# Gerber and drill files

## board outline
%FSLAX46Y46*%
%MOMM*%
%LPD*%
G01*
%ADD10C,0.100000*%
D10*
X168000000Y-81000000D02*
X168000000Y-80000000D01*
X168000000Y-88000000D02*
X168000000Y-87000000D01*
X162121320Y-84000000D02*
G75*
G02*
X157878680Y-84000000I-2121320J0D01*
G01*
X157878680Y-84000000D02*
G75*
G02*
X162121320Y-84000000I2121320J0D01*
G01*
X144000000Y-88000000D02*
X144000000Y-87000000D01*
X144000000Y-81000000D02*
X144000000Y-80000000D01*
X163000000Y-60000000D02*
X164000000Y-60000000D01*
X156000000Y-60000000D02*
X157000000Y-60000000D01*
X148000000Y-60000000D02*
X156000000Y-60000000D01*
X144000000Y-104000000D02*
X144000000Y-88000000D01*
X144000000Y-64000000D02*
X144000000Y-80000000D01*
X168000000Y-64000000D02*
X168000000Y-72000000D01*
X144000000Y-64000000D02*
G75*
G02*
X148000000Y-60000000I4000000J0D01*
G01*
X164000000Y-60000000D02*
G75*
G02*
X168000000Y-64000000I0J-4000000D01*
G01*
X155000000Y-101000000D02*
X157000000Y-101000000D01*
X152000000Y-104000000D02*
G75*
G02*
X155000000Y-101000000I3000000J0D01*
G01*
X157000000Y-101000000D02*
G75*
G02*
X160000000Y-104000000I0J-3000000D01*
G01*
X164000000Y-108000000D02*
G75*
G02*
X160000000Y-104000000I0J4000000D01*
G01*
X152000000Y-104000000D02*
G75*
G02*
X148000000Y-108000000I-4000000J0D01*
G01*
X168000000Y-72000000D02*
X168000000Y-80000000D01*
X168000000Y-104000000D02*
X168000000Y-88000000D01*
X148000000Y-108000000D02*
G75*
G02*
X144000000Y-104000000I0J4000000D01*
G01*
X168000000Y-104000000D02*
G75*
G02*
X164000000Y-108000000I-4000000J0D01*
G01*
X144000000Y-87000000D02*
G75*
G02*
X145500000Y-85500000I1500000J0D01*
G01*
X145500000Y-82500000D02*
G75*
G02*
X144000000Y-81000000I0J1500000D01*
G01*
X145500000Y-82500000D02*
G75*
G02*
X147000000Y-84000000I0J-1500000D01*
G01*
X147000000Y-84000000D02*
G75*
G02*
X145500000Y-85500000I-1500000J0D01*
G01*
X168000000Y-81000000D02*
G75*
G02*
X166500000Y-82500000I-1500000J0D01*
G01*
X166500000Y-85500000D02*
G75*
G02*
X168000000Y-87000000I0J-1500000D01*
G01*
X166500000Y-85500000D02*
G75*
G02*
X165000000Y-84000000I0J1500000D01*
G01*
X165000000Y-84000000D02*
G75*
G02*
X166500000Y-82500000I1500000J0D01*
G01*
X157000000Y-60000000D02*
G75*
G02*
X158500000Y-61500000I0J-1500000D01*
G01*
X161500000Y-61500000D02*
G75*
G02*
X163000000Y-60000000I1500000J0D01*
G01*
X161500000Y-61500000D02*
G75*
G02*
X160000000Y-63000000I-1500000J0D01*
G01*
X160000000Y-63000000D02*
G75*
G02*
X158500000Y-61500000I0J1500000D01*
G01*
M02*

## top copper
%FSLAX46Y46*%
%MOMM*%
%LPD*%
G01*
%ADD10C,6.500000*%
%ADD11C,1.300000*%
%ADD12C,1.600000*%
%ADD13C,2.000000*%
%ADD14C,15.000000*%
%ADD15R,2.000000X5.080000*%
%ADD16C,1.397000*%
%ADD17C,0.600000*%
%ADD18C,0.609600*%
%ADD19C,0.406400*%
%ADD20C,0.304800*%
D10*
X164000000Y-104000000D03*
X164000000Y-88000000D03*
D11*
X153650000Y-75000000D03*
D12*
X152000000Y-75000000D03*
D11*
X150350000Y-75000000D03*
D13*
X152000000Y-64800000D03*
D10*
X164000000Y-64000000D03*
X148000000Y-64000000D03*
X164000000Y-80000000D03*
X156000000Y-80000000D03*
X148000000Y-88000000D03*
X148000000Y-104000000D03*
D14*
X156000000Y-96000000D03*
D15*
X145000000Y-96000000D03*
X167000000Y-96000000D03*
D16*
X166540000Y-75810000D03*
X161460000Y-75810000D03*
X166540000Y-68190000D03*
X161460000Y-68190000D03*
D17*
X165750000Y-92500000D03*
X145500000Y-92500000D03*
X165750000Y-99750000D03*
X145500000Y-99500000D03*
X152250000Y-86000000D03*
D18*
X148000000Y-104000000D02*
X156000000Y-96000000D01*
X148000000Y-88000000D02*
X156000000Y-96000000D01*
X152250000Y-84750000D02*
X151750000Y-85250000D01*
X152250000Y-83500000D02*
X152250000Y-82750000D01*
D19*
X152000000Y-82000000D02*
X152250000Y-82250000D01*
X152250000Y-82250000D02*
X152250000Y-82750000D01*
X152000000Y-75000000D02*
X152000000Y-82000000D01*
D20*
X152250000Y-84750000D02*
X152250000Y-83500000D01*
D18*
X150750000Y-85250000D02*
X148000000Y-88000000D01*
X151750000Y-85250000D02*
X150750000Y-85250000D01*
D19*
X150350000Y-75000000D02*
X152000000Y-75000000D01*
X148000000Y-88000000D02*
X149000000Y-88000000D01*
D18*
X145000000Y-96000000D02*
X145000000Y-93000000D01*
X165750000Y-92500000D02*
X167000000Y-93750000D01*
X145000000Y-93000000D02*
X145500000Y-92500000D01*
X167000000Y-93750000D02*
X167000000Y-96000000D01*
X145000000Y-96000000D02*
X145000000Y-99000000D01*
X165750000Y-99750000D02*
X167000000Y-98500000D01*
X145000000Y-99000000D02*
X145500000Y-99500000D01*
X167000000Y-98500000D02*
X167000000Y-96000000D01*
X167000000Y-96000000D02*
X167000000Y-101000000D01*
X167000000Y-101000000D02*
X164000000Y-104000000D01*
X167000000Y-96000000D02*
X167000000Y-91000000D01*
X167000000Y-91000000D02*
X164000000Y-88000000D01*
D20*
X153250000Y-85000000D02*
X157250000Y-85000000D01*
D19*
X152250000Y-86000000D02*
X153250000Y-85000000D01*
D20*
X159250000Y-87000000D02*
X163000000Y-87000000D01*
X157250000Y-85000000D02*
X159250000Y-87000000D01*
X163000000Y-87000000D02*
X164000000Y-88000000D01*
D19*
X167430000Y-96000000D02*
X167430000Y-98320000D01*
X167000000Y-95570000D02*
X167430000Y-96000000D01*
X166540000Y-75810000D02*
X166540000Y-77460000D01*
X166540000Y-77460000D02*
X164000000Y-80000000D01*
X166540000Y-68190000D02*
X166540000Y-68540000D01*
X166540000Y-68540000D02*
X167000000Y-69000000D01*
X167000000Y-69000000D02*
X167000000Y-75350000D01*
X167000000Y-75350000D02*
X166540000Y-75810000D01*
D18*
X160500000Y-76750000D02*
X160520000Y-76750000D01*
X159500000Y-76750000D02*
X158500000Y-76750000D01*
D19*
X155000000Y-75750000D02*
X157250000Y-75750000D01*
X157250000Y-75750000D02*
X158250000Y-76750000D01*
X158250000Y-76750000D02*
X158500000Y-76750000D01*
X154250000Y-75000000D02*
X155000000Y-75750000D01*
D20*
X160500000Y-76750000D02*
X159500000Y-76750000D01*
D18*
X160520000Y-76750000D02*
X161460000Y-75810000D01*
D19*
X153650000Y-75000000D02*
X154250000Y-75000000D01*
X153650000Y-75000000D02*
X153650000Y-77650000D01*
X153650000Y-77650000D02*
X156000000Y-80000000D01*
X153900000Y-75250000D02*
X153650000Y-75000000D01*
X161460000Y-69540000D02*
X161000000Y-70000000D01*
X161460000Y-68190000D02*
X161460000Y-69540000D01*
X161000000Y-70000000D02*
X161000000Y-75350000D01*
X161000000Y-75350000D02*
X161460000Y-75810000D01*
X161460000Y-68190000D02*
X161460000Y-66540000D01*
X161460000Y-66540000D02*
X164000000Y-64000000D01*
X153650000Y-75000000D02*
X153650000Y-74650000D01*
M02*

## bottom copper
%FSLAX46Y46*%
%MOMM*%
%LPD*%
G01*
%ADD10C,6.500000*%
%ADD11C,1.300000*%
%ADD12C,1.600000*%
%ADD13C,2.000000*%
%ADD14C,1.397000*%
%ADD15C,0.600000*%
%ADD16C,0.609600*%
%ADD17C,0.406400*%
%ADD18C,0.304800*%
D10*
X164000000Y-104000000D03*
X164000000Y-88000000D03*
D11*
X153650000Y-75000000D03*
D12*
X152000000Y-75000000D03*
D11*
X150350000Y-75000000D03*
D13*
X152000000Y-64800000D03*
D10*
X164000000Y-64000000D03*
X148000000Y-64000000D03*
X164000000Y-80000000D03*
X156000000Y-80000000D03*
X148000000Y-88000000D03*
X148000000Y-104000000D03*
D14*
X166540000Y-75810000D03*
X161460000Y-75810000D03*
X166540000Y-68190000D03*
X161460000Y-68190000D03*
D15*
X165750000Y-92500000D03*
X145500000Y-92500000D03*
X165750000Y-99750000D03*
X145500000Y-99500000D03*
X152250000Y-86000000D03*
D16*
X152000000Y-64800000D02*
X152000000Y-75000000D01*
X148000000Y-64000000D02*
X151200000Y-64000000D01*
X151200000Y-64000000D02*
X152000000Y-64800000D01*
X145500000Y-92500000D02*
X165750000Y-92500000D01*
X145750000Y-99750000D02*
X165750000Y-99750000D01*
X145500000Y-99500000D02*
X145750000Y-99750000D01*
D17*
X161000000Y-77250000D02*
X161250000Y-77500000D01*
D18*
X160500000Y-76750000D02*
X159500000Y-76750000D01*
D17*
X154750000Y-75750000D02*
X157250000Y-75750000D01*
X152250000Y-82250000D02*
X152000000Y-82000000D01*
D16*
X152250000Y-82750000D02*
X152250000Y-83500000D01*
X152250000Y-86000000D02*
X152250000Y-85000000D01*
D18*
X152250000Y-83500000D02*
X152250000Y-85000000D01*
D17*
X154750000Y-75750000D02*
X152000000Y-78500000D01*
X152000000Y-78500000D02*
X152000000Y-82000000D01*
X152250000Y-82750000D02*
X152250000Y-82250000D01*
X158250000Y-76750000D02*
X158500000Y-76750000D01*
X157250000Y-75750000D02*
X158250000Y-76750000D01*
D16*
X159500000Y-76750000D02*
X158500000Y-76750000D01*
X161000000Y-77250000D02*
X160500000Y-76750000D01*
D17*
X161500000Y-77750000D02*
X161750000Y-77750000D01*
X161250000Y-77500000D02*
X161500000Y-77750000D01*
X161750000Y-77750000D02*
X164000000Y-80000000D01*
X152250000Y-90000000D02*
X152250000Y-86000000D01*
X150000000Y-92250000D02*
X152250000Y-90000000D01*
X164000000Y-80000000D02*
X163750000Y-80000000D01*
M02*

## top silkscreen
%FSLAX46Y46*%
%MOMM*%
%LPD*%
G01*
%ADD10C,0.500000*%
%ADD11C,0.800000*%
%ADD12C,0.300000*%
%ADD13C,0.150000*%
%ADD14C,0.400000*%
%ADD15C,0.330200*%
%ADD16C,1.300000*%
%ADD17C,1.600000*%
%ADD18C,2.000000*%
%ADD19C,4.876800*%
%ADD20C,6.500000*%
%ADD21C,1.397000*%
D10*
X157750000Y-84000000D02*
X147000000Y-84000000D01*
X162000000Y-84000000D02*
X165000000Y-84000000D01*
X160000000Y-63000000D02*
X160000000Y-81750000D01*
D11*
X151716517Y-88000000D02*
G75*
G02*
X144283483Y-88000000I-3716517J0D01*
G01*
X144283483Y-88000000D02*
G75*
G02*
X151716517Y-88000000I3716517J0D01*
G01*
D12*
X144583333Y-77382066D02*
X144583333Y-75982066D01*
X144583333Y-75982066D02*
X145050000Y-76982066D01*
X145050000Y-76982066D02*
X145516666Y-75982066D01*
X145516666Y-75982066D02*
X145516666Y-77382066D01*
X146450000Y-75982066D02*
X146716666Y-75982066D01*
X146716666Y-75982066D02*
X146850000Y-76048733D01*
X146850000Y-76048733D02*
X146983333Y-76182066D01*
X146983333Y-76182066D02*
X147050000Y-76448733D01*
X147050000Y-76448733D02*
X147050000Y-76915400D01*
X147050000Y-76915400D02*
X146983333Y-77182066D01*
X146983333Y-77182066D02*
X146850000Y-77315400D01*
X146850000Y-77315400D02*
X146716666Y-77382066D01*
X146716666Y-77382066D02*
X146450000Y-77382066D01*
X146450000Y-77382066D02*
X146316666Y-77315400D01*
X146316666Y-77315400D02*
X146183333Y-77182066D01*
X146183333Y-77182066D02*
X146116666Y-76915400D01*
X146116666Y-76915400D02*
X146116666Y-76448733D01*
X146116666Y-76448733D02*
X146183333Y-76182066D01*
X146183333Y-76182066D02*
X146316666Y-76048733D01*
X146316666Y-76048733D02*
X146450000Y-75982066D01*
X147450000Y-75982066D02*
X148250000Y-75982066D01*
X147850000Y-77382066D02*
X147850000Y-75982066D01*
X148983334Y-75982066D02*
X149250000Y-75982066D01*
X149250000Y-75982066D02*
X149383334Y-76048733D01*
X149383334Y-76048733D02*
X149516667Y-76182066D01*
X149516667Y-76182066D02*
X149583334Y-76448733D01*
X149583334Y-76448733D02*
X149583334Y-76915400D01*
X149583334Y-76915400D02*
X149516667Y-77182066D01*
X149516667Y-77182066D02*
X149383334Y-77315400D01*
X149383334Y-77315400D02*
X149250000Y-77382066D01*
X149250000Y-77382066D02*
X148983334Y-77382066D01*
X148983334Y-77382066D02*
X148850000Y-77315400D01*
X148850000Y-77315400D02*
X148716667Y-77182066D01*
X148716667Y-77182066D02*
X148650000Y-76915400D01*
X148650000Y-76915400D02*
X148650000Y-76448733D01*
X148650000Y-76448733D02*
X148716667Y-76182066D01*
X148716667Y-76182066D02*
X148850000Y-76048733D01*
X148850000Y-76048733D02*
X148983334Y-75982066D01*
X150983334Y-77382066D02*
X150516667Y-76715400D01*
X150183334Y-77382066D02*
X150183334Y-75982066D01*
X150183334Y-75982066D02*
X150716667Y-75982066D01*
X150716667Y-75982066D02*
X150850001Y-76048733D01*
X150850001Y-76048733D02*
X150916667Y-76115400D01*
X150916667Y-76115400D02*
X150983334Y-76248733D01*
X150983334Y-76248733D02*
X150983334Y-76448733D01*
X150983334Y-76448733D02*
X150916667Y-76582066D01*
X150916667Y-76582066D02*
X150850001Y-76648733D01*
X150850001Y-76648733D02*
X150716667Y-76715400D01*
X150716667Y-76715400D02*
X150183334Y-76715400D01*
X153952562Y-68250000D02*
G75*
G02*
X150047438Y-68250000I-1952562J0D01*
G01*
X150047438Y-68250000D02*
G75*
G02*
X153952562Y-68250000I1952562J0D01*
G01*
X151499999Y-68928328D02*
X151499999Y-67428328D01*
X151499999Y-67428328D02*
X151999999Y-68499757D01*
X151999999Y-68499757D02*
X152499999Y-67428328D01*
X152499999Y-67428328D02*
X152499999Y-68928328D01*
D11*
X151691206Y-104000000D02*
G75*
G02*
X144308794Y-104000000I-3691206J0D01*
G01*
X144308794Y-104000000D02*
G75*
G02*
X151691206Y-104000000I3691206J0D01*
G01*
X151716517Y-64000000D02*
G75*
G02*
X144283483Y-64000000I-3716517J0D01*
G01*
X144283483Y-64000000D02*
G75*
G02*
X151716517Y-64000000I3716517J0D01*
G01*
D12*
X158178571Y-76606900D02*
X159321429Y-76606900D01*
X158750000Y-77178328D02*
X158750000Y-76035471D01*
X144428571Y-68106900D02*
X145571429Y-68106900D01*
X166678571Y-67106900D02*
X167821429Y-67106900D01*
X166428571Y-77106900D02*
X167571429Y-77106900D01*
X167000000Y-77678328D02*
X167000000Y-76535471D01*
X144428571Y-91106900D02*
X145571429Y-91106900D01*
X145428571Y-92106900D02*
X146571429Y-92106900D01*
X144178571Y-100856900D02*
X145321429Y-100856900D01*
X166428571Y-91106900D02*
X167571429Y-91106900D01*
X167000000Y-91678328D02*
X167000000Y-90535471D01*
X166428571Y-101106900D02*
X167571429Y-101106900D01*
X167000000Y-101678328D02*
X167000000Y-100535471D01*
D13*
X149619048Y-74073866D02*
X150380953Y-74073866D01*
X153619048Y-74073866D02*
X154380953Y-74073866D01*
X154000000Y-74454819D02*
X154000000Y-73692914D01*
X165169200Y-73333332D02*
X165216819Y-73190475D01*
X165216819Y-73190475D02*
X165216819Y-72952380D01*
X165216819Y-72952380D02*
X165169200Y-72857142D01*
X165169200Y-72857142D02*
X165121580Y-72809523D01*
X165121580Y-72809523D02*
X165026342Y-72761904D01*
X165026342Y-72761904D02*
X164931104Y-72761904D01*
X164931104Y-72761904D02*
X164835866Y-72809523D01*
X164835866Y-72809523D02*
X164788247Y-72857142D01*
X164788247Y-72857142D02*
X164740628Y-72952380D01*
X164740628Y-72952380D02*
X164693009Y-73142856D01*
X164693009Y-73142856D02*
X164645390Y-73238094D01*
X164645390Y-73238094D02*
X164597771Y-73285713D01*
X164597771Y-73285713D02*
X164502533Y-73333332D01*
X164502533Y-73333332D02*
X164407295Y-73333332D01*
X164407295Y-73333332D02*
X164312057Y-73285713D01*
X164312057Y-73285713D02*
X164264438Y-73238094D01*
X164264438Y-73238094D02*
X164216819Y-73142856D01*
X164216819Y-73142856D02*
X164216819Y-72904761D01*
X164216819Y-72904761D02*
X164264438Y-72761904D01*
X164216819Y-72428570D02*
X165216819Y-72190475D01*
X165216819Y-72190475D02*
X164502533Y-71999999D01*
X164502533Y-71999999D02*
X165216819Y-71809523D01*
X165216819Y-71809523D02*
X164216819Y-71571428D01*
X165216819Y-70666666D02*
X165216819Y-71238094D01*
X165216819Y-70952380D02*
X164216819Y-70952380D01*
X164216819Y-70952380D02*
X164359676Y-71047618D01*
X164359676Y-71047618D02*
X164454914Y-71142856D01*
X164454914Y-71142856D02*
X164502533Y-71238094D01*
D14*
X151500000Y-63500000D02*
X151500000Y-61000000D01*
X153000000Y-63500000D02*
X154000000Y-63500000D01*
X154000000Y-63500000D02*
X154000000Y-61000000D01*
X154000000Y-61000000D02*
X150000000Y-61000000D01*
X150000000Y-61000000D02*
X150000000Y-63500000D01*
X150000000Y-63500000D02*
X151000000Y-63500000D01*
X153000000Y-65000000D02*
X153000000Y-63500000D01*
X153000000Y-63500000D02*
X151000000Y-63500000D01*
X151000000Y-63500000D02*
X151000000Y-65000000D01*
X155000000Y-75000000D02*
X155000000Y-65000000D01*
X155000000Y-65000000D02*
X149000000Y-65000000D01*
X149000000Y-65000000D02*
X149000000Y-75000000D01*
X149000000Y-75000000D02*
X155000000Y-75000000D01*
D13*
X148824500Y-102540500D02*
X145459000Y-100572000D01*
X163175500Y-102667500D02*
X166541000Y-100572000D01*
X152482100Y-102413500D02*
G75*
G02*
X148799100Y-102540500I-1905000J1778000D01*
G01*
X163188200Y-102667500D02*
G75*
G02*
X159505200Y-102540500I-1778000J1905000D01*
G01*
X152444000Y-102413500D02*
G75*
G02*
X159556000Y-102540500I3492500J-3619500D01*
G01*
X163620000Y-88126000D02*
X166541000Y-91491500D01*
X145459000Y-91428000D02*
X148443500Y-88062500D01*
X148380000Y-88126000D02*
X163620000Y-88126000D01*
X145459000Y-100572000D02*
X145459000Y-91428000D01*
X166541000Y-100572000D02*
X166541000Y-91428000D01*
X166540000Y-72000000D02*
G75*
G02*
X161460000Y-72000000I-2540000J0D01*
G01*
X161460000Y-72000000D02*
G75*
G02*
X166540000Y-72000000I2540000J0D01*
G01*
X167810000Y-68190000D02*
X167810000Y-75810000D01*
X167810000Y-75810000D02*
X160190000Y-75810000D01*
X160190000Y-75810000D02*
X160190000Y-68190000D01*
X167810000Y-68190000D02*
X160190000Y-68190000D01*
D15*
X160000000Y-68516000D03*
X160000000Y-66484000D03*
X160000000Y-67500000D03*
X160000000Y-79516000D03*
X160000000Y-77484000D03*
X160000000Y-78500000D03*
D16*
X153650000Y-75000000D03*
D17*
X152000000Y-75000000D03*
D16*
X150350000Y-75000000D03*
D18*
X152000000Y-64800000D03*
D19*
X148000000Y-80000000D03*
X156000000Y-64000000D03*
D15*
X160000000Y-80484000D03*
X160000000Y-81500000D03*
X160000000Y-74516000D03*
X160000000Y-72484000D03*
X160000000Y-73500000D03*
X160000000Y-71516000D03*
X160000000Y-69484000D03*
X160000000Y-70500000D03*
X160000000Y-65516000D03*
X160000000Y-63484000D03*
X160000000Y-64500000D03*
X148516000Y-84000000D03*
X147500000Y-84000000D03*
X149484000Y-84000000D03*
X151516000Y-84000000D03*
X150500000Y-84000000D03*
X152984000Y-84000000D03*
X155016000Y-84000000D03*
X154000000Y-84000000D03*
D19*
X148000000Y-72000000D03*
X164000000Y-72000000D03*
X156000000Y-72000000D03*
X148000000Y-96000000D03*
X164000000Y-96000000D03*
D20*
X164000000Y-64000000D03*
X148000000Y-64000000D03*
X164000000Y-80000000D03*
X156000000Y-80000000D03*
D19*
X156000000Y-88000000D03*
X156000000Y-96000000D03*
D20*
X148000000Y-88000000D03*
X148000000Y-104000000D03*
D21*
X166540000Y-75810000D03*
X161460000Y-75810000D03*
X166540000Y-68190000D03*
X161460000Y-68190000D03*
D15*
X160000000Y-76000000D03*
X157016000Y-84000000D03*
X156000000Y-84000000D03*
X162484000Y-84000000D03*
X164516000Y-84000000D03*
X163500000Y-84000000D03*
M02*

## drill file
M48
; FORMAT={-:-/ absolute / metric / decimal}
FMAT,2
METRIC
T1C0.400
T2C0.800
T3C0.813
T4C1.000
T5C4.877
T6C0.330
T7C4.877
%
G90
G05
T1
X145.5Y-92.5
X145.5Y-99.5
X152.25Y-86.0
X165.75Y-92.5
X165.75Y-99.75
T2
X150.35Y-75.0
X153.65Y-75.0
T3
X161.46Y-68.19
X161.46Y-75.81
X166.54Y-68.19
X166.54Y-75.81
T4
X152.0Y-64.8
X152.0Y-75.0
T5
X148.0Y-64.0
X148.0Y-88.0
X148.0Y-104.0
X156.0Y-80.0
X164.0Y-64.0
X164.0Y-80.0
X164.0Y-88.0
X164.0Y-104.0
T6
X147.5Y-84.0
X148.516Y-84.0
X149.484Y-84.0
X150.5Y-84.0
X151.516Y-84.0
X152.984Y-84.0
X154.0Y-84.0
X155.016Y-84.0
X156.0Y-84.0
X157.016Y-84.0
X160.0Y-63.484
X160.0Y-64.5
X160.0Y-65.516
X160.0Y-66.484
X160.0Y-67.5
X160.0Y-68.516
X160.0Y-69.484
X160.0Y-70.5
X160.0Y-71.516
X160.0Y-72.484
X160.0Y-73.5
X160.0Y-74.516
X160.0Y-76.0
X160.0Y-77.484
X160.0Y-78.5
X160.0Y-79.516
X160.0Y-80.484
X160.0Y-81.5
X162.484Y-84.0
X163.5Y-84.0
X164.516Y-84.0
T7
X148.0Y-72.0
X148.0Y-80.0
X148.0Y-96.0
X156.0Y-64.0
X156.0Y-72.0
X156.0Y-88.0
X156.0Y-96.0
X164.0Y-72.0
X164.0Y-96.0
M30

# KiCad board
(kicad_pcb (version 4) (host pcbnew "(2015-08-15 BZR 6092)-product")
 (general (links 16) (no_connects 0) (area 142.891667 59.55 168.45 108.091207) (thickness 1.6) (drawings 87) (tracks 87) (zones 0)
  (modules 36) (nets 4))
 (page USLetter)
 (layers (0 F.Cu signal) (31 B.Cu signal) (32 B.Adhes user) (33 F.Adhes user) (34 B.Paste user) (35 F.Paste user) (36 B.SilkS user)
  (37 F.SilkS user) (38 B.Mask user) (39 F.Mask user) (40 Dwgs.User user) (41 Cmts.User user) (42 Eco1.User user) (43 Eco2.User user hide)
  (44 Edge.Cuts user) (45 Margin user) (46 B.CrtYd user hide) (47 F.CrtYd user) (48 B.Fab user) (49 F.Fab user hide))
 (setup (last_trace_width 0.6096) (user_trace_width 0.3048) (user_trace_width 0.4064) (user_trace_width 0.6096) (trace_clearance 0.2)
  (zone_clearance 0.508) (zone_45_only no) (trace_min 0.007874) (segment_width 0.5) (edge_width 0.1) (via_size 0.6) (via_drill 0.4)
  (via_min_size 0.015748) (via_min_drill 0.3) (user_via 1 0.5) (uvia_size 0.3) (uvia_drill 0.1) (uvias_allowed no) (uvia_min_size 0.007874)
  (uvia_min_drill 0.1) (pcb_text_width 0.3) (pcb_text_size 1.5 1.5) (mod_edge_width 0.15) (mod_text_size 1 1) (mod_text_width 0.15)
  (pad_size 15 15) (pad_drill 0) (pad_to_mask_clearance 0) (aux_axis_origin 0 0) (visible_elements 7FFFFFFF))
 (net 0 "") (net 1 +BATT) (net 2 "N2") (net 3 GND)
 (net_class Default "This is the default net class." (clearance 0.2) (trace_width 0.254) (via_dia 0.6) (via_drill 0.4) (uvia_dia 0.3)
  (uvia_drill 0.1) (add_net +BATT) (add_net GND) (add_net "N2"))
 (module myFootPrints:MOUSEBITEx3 (layer F.Cu) (at 160 67.5 90)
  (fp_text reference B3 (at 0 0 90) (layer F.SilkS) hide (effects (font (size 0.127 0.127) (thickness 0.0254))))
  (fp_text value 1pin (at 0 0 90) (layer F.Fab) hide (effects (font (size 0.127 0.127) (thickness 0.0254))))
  (pad "" np_thru_hole circle (at -1.016 0 90) (size 0.3302 0.3302) (drill 0.3302) (layers *.Cu *.Mask F.SilkS))
  (pad "" np_thru_hole circle (at 1.016 0 90) (size 0.3302 0.3302) (drill 0.3302) (layers *.Cu *.Mask F.SilkS))
  (pad "" np_thru_hole circle (at 0 0 90) (size 0.3302 0.3302) (drill 0.3302) (layers *.Cu *.Mask F.SilkS)))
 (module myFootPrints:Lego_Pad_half (layer F.Cu) (at 164 104 180)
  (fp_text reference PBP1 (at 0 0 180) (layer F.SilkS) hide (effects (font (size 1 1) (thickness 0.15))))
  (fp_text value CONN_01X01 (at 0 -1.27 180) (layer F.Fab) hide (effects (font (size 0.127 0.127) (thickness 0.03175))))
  (pad 1 thru_hole circle (at 0 0 180) (size 6.5 6.5) (drill 4.8768) (layers *.Cu B.SilkS B.Mask) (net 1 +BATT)))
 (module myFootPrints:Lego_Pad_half (layer F.Cu) (at 164 88 270)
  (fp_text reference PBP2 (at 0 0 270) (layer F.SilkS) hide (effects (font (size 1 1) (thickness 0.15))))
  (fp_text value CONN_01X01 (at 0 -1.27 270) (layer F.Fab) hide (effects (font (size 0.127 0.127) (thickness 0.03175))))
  (pad 1 thru_hole circle (at 0 0 270) (size 6.5 6.5) (drill 4.8768) (layers *.Cu B.SilkS B.Mask) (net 1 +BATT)))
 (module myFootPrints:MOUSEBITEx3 (layer F.Cu) (at 160 78.5 90)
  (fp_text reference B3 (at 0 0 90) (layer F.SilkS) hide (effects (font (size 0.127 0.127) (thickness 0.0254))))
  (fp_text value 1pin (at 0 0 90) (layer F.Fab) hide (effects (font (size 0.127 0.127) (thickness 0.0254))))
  (pad "" np_thru_hole circle (at -1.016 0 90) (size 0.3302 0.3302) (drill 0.3302) (layers *.Cu *.Mask F.SilkS))
  (pad "" np_thru_hole circle (at 1.016 0 90) (size 0.3302 0.3302) (drill 0.3302) (layers *.Cu *.Mask F.SilkS))
  (pad "" np_thru_hole circle (at 0 0 90) (size 0.3302 0.3302) (drill 0.3302) (layers *.Cu *.Mask F.SilkS)))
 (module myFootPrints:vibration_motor (layer F.Cu) (at 152 70 180)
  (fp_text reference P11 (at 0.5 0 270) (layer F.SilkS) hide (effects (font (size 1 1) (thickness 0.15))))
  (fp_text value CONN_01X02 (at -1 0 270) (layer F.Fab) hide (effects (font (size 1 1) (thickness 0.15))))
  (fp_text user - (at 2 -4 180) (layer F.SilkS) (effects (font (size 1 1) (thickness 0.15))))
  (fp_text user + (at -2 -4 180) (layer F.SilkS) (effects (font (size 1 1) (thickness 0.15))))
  (fp_line (start 0.5 6.5) (end 0.5 9) (layer F.SilkS) (width 0.4))
  (fp_line (start -1 6.5) (end -2 6.5) (layer F.SilkS) (width 0.4))
  (fp_line (start -2 6.5) (end -2 9) (layer F.SilkS) (width 0.4)) (fp_line (start -2 9) (end 2 9) (layer F.SilkS) (width 0.4))
  (fp_line (start 2 9) (end 2 6.5) (layer F.SilkS) (width 0.4))
  (fp_line (start 2 6.5) (end 1 6.5) (layer F.SilkS) (width 0.4))
  (fp_line (start -1 5) (end -1 6.5) (layer F.SilkS) (width 0.4))
  (fp_line (start -1 6.5) (end 1 6.5) (layer F.SilkS) (width 0.4))
  (fp_line (start 1 6.5) (end 1 5) (layer F.SilkS) (width 0.4))
  (fp_line (start -3 -5) (end -3 5) (layer F.SilkS) (width 0.4)) (fp_line (start -3 5) (end 3 5) (layer F.SilkS) (width 0.4))
  (fp_line (start 3 5) (end 3 -5) (layer F.SilkS) (width 0.4))
  (fp_line (start 3 -5) (end -3 -5) (layer F.SilkS) (width 0.4))
  (pad 1 thru_hole circle (at -1.65 -5 180) (size 1.3 1.3) (drill 0.8) (layers *.Cu *.Mask F.SilkS) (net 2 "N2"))
  (pad 2 thru_hole circle (at 0 -5 180) (size 1.6 1.6) (drill 1) (layers *.Cu *.Mask F.SilkS) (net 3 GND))
  (pad 2 thru_hole circle (at 1.65 -5 180) (size 1.3 1.3) (drill 0.8) (layers *.Cu *.Mask F.SilkS) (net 3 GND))
  (pad 2 thru_hole circle (at 0 5.2 180) (size 2 2) (drill 1) (layers *.Cu *.Mask F.SilkS) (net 3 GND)))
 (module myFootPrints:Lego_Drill (layer F.Cu) (at 148 80)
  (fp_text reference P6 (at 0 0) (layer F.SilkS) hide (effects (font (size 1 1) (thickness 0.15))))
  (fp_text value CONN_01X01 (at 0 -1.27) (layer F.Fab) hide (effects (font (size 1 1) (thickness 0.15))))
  (pad "" np_thru_hole circle (at 0 0) (size 4.8768 4.8768) (drill 4.8768) (layers *.Cu *.Mask F.SilkS)))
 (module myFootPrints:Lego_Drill (layer F.Cu) (at 156 64)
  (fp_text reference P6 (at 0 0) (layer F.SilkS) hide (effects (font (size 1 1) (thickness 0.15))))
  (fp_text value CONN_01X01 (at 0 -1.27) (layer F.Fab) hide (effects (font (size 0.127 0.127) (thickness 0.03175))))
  (pad "" np_thru_hole circle (at 0 0) (size 4.8768 4.8768) (drill 4.8768) (layers *.Cu *.Mask F.SilkS)))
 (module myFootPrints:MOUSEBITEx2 (layer F.Cu) (at 160 81.5 90)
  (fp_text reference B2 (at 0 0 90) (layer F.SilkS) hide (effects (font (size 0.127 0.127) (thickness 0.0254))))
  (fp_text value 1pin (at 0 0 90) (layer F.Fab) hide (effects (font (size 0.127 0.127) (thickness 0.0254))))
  (pad "" np_thru_hole circle (at 1.016 0 90) (size 0.3302 0.3302) (drill 0.3302) (layers *.Cu *.Mask F.SilkS))
  (pad "" np_thru_hole circle (at 0 0 90) (size 0.3302 0.3302) (drill 0.3302) (layers *.Cu *.Mask F.SilkS)))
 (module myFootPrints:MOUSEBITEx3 (layer F.Cu) (at 160 73.5 90)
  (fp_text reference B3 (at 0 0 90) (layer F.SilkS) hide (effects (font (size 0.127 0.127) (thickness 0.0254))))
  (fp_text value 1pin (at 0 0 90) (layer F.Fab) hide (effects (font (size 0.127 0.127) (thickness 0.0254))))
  (pad "" np_thru_hole circle (at -1.016 0 90) (size 0.3302 0.3302) (drill 0.3302) (layers *.Cu *.Mask F.SilkS))
  (pad "" np_thru_hole circle (at 1.016 0 90) (size 0.3302 0.3302) (drill 0.3302) (layers *.Cu *.Mask F.SilkS))
  (pad "" np_thru_hole circle (at 0 0 90) (size 0.3302 0.3302) (drill 0.3302) (layers *.Cu *.Mask F.SilkS)))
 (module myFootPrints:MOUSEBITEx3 (layer F.Cu) (at 160 70.5 90)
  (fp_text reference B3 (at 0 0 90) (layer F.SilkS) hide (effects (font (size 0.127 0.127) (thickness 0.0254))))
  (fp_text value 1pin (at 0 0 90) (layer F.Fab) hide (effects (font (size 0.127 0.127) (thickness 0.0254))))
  (pad "" np_thru_hole circle (at -1.016 0 90) (size 0.3302 0.3302) (drill 0.3302) (layers *.Cu *.Mask F.SilkS))
  (pad "" np_thru_hole circle (at 1.016 0 90) (size 0.3302 0.3302) (drill 0.3302) (layers *.Cu *.Mask F.SilkS))
  (pad "" np_thru_hole circle (at 0 0 90) (size 0.3302 0.3302) (drill 0.3302) (layers *.Cu *.Mask F.SilkS)))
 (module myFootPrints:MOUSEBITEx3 (layer F.Cu) (at 160 64.5 90)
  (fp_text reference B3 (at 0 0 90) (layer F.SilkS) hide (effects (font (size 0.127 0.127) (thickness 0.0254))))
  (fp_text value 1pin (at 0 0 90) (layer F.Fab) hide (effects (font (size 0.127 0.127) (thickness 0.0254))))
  (pad "" np_thru_hole circle (at -1.016 0 90) (size 0.3302 0.3302) (drill 0.3302) (layers *.Cu *.Mask F.SilkS))
  (pad "" np_thru_hole circle (at 1.016 0 90) (size 0.3302 0.3302) (drill 0.3302) (layers *.Cu *.Mask F.SilkS))
  (pad "" np_thru_hole circle (at 0 0 90) (size 0.3302 0.3302) (drill 0.3302) (layers *.Cu *.Mask F.SilkS)))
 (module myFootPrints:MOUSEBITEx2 (layer F.Cu) (at 147.5 84)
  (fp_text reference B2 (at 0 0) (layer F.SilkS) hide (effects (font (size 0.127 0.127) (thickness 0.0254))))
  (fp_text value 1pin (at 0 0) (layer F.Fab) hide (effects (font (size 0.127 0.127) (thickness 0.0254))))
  (pad "" np_thru_hole circle (at 1.016 0) (size 0.3302 0.3302) (drill 0.3302) (layers *.Cu *.Mask F.SilkS))
  (pad "" np_thru_hole circle (at 0 0) (size 0.3302 0.3302) (drill 0.3302) (layers *.Cu *.Mask F.SilkS)))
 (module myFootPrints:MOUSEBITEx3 (layer F.Cu) (at 150.5 84)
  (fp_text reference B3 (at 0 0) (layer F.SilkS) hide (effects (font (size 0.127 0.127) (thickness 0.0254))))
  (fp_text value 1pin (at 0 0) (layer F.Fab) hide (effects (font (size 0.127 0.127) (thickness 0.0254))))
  (pad "" np_thru_hole circle (at -1.016 0) (size 0.3302 0.3302) (drill 0.3302) (layers *.Cu *.Mask F.SilkS))
  (pad "" np_thru_hole circle (at 1.016 0) (size 0.3302 0.3302) (drill 0.3302) (layers *.Cu *.Mask F.SilkS))
  (pad "" np_thru_hole circle (at 0 0) (size 0.3302 0.3302) (drill 0.3302) (layers *.Cu *.Mask F.SilkS)))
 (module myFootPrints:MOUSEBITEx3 (layer F.Cu) (at 154 84)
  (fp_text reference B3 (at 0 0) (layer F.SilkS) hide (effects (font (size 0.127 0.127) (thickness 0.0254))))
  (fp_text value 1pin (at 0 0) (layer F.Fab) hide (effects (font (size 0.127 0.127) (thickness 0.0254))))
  (pad "" np_thru_hole circle (at -1.016 0) (size 0.3302 0.3302) (drill 0.3302) (layers *.Cu *.Mask F.SilkS))
  (pad "" np_thru_hole circle (at 1.016 0) (size 0.3302 0.3302) (drill 0.3302) (layers *.Cu *.Mask F.SilkS))
  (pad "" np_thru_hole circle (at 0 0) (size 0.3302 0.3302) (drill 0.3302) (layers *.Cu *.Mask F.SilkS)))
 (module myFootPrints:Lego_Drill (layer F.Cu) (at 148 72)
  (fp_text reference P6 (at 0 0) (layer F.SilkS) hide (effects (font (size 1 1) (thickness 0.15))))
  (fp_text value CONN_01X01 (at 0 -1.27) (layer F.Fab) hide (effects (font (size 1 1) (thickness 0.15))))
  (pad "" np_thru_hole circle (at 0 0) (size 4.8768 4.8768) (drill 4.8768) (layers *.Cu *.Mask F.SilkS)))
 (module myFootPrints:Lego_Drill (layer F.Cu) (at 164 72)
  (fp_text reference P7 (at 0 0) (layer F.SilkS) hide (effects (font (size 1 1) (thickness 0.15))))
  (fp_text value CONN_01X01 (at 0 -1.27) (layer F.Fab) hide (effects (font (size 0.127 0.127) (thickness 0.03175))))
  (pad "" np_thru_hole circle (at 0 0) (size 4.8768 4.8768) (drill 4.8768) (layers *.Cu *.Mask F.SilkS)))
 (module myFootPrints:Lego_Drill (layer F.Cu) (at 156 72)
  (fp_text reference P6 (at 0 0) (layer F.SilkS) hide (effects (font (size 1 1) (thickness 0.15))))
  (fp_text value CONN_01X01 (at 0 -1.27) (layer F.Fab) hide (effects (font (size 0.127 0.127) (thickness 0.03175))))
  (pad "" np_thru_hole circle (at 0 0) (size 4.8768 4.8768) (drill 4.8768) (layers *.Cu *.Mask F.SilkS)))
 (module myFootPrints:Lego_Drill (layer F.Cu) (at 148 96)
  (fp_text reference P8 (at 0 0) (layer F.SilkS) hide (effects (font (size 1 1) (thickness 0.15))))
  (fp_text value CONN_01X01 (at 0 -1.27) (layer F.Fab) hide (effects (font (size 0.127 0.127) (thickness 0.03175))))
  (pad "" np_thru_hole circle (at 0 0) (size 4.8768 4.8768) (drill 4.8768) (layers *.Cu *.Mask F.SilkS)))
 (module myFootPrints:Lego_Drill (layer F.Cu) (at 164 96)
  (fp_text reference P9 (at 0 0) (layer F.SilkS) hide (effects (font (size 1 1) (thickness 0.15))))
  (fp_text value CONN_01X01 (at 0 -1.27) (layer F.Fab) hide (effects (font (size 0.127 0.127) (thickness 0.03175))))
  (pad "" np_thru_hole circle (at 0 0) (size 4.8768 4.8768) (drill 4.8768) (layers *.Cu *.Mask F.SilkS)))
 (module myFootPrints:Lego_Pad (layer F.Cu) (at 164 64)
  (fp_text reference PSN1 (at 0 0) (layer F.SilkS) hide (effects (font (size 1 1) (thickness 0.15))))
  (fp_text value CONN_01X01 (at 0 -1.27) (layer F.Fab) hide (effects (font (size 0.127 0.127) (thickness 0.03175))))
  (pad 1 thru_hole circle (at 0 0) (size 6.5 6.5) (drill 4.8768) (layers *.Cu *.Mask F.SilkS) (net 2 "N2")))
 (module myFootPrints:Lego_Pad (layer F.Cu) (at 148 64)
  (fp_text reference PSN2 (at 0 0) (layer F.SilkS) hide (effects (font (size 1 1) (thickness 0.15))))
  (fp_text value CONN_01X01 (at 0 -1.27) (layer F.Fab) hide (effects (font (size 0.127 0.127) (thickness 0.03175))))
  (pad 1 thru_hole circle (at 0 0) (size 6.5 6.5) (drill 4.8768) (layers *.Cu *.Mask F.SilkS) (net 3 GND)))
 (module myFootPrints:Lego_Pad (layer F.Cu) (at 164 80)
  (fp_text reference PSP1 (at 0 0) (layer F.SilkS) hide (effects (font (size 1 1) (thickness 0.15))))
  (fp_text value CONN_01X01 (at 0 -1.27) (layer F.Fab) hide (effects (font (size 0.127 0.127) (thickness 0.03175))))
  (pad 1 thru_hole circle (at 0 0) (size 6.5 6.5) (drill 4.8768) (layers *.Cu *.Mask F.SilkS) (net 1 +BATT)))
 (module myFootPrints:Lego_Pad (layer F.Cu) (at 156 80)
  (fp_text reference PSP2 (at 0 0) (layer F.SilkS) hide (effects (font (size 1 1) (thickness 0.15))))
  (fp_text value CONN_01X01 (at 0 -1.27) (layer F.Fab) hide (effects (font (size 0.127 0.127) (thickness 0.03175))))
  (pad 1 thru_hole circle (at 0 0) (size 6.5 6.5) (drill 4.8768) (layers *.Cu *.Mask F.SilkS) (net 2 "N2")))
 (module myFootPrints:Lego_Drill (layer F.Cu) (at 156 88)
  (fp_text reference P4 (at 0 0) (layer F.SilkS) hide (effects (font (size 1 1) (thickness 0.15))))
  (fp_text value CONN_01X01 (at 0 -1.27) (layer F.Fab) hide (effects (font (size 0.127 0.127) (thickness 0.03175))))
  (pad "" np_thru_hole circle (at 0 0) (size 4.8768 4.8768) (drill 4.8768) (layers *.Cu *.Mask F.SilkS)))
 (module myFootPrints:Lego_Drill (layer F.Cu) (at 156 96)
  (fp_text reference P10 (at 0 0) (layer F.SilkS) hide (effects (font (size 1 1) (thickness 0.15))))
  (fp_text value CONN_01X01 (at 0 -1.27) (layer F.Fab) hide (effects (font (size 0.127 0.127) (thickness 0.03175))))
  (pad "" np_thru_hole circle (at 0 0) (size 4.8768 4.8768) (drill 4.8768) (layers *.Cu *.Mask F.SilkS)))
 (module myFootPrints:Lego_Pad (layer F.Cu) (at 148 88)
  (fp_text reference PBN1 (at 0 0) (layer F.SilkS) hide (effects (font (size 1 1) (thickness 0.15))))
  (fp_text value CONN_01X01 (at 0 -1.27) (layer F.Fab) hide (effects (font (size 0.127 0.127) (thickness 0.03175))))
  (pad 1 thru_hole circle (at 0 0) (size 6.5 6.5) (drill 4.8768) (layers *.Cu *.Mask F.SilkS) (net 3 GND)))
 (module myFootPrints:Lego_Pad (layer F.Cu) (at 148 104)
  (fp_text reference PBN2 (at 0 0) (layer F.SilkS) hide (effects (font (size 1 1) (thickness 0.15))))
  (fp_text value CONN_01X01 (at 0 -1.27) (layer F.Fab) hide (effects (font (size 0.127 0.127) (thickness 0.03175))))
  (pad 1 thru_hole circle (at 0 0) (size 6.5 6.5) (drill 4.8768) (layers *.Cu *.Mask F.SilkS) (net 3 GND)))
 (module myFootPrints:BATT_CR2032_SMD (layer F.Cu) (at 156 96)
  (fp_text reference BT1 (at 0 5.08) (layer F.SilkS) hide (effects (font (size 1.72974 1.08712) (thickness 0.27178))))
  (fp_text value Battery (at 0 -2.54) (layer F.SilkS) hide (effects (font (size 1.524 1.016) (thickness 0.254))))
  (fp_line (start -7.1755 6.5405) (end -10.541 4.572) (layer F.SilkS) (width 0.15))
  (fp_line (start 7.1755 6.6675) (end 10.541 4.572) (layer F.SilkS) (width 0.15))
  (fp_arc (start -5.4229 4.6355) (end -3.5179 6.4135) (angle 90) (layer F.SilkS) (width 0.15))
  (fp_arc (start 5.4102 4.7625) (end 7.1882 6.6675) (angle 90) (layer F.SilkS) (width 0.15))
  (fp_arc (start -0.0635 10.033) (end -3.556 6.4135) (angle 90) (layer F.SilkS) (width 0.15))
  (fp_line (start 7.62 -7.874) (end 10.541 -4.5085) (layer F.SilkS) (width 0.15))
  (fp_line (start -10.541 -4.572) (end -7.5565 -7.9375) (layer F.SilkS) (width 0.15))
  (fp_line (start -7.62 -7.874) (end 7.62 -7.874) (layer F.SilkS) (width 0.15))
  (fp_line (start -10.541 4.572) (end -10.541 -4.572) (layer F.SilkS) (width 0.15))
  (fp_line (start 10.541 4.572) (end 10.541 -4.572) (layer F.SilkS) (width 0.15))
  (pad 2 smd circle (at 0 0) (size 15 15) (layers F.Cu F.Paste F.Mask) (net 3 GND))
  (pad 1 smd rect (at -11 0) (size 2 5.08) (layers F.Cu F.Paste F.Mask) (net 1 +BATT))
  (pad 1 smd rect (at 11 0) (size 2 5.08) (layers F.Cu F.Paste F.Mask) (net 1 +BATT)))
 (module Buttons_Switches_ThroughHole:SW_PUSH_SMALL (layer F.Cu) (at 164 72 270)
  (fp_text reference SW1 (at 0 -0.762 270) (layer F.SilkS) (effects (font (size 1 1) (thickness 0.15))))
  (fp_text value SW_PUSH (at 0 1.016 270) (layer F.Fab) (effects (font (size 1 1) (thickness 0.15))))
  (fp_circle (center 0 0) (end 0 -2.54) (layer F.SilkS) (width 0.15))
  (fp_line (start -3.81 -3.81) (end 3.81 -3.81) (layer F.SilkS) (width 0.15))
  (fp_line (start 3.81 -3.81) (end 3.81 3.81) (layer F.SilkS) (width 0.15))
  (fp_line (start 3.81 3.81) (end -3.81 3.81) (layer F.SilkS) (width 0.15))
  (fp_line (start -3.81 -3.81) (end -3.81 3.81) (layer F.SilkS) (width 0.15))
  (pad 1 thru_hole circle (at 3.81 -2.54 270) (size 1.397 1.397) (drill 0.8128) (layers *.Cu *.Mask F.SilkS) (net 1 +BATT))
  (pad 2 thru_hole circle (at 3.81 2.54 270) (size 1.397 1.397) (drill 0.8128) (layers *.Cu *.Mask F.SilkS) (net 2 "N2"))
  (pad 1 thru_hole circle (at -3.81 -2.54 270) (size 1.397 1.397) (drill 0.8128) (layers *.Cu *.Mask F.SilkS) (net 1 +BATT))
  (pad 2 thru_hole circle (at -3.81 2.54 270) (size 1.397 1.397) (drill 0.8128) (layers *.Cu *.Mask F.SilkS) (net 2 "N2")))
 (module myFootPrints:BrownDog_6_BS (layer F.Cu) (at 160.4 92.8)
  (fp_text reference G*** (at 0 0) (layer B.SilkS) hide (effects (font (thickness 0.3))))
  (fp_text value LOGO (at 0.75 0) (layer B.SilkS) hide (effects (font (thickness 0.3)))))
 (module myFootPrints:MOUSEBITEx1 (layer F.Cu) (at 160 76)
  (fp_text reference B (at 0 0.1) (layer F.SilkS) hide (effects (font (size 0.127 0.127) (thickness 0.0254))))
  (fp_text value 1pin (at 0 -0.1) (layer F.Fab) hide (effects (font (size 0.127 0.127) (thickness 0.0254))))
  (pad "" np_thru_hole circle (at 0 0) (size 0.3302 0.3302) (drill 0.3302) (layers *.Cu *.Mask F.SilkS)))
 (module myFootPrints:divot (layer F.Cu) (at 144 84 90)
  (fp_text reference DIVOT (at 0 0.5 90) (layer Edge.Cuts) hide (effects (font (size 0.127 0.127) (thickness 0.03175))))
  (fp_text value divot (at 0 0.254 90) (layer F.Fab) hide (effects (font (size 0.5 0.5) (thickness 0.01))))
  (fp_arc (start -3 1.5) (end -3 0) (angle 90) (layer Edge.Cuts) (width 0.1))
  (fp_arc (start 3 1.5) (end 1.5 1.5) (angle 90) (layer Edge.Cuts) (width 0.1))
  (fp_arc (start 0 1.5) (end 1.5 1.5) (angle 90) (layer Edge.Cuts) (width 0.1))
  (fp_arc (start 0 1.5) (end 0 3) (angle 90) (layer Edge.Cuts) (width 0.1)))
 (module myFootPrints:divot (layer F.Cu) (at 168 84 270)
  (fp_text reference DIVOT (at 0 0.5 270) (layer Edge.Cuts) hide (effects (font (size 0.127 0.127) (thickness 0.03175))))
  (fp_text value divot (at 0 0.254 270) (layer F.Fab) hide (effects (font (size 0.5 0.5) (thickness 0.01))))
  (fp_arc (start -3 1.5) (end -3 0) (angle 90) (layer Edge.Cuts) (width 0.1))
  (fp_arc (start 3 1.5) (end 1.5 1.5) (angle 90) (layer Edge.Cuts) (width 0.1))
  (fp_arc (start 0 1.5) (end 1.5 1.5) (angle 90) (layer Edge.Cuts) (width 0.1))
  (fp_arc (start 0 1.5) (end 0 3) (angle 90) (layer Edge.Cuts) (width 0.1)))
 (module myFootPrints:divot (layer F.Cu) (at 160 60)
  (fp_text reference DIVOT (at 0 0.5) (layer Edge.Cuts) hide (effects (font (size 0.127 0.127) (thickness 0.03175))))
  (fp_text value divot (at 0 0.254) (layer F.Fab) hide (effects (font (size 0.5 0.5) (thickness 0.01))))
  (fp_arc (start -3 1.5) (end -3 0) (angle 90) (layer Edge.Cuts) (width 0.1))
  (fp_arc (start 3 1.5) (end 1.5 1.5) (angle 90) (layer Edge.Cuts) (width 0.1))
  (fp_arc (start 0 1.5) (end 1.5 1.5) (angle 90) (layer Edge.Cuts) (width 0.1))
  (fp_arc (start 0 1.5) (end 0 3) (angle 90) (layer Edge.Cuts) (width 0.1)))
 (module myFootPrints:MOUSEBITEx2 (layer F.Cu) (at 156 84)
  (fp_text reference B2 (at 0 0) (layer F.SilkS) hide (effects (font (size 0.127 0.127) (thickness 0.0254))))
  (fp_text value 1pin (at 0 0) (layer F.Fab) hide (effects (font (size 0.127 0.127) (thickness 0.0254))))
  (pad "" np_thru_hole circle (at 1.016 0) (size 0.3302 0.3302) (drill 0.3302) (layers *.Cu *.Mask F.SilkS))
  (pad "" np_thru_hole circle (at 0 0) (size 0.3302 0.3302) (drill 0.3302) (layers *.Cu *.Mask F.SilkS)))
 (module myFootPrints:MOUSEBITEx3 (layer F.Cu) (at 163.5 84)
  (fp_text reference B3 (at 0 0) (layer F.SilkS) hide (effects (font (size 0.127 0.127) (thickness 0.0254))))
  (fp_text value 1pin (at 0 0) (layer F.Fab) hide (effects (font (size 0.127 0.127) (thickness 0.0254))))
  (pad "" np_thru_hole circle (at -1.016 0) (size 0.3302 0.3302) (drill 0.3302) (layers *.Cu *.Mask F.SilkS))
  (pad "" np_thru_hole circle (at 1.016 0) (size 0.3302 0.3302) (drill 0.3302) (layers *.Cu *.Mask F.SilkS))
  (pad "" np_thru_hole circle (at 0 0) (size 0.3302 0.3302) (drill 0.3302) (layers *.Cu *.Mask F.SilkS)))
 (gr_line (start 157.75 84) (end 147 84) (angle 90) (layer F.SilkS) (width 0.5))
 (gr_line (start 162 84) (end 165 84) (angle 90) (layer F.SilkS) (width 0.5))
 (gr_line (start 160 63) (end 160 81.75) (angle 90) (layer F.SilkS) (width 0.5))
 (gr_line (start 168 81) (end 168 80) (angle 90) (layer Edge.Cuts) (width 0.1))
 (gr_line (start 168 88) (end 168 87) (angle 90) (layer Edge.Cuts) (width 0.1))
 (gr_circle (center 160 84) (end 158.5 82.5) (layer Edge.Cuts) (width 0.1))
 (gr_line (start 144 88) (end 144 87) (angle 90) (layer Edge.Cuts) (width 0.1))
 (gr_line (start 144 81) (end 144 80) (angle 90) (layer Edge.Cuts) (width 0.1))
 (gr_circle (center 148 88) (end 144.5 86.75) (layer F.SilkS) (width 0.8))
 (gr_line (start 163 60) (end 164 60) (angle 90) (layer Edge.Cuts) (width 0.1))
 (gr_line (start 156 60) (end 157 60) (angle 90) (layer Edge.Cuts) (width 0.1))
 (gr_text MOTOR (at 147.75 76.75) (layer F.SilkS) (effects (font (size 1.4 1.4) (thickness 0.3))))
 (gr_circle (center 152 68.25) (end 150.5 67) (layer F.SilkS) (width 0.3))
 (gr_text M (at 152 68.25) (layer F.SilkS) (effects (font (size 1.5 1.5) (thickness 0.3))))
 (gr_circle (center 148 104) (end 146.25 100.75) (layer F.SilkS) (width 0.8))
 (gr_circle (center 148 64) (end 146.75 60.5) (layer F.SilkS) (width 0.8))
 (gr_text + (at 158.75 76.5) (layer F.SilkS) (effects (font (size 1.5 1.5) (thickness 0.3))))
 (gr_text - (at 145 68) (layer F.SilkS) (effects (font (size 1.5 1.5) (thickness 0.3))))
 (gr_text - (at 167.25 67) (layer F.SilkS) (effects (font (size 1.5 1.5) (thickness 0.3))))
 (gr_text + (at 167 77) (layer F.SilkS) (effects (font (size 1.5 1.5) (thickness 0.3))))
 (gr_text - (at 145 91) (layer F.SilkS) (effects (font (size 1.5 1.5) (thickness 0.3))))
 (gr_line (start 148 60) (end 156 60) (angle 90) (layer Edge.Cuts) (width 0.1))
 (gr_line (start 144 104) (end 144 88) (angle 90) (layer Edge.Cuts) (width 0.1))
 (gr_line (start 144 64) (end 144 80) (angle 90) (layer Edge.Cuts) (width 0.1))
 (gr_line (start 168 64) (end 168 72) (angle 90) (layer Edge.Cuts) (width 0.1))
 (gr_arc (start 148 64) (end 144 64) (angle 90) (layer Edge.Cuts) (width 0.1))
 (gr_arc (start 164 64) (end 164 60) (angle 90) (layer Edge.Cuts) (width 0.1))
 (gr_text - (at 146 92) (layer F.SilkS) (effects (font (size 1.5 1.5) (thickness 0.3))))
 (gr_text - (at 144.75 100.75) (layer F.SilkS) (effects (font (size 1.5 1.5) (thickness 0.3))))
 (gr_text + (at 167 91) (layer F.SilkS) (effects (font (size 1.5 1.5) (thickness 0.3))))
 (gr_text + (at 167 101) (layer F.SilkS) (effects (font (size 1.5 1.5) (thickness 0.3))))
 (gr_line (start 155 101) (end 157 101) (angle 90) (layer Edge.Cuts) (width 0.1))
 (gr_arc (start 155 104) (end 152 104) (angle 90) (layer Edge.Cuts) (width 0.1))
 (gr_arc (start 157 104) (end 157 101) (angle 90) (layer Edge.Cuts) (width 0.1))
 (gr_arc (start 164 104) (end 164 108) (angle 90) (layer Edge.Cuts) (width 0.1))
 (gr_arc (start 148 104) (end 152 104) (angle 90) (layer Edge.Cuts) (width 0.1))
 (gr_line (start 168 72) (end 168 80) (angle 90) (layer Edge.Cuts) (width 0.1))
 (gr_line (start 168 104) (end 168 88) (angle 90) (layer Edge.Cuts) (width 0.1))
 (gr_arc (start 148 104) (end 148 108) (angle 90) (layer Edge.Cuts) (width 0.1))
 (gr_arc (start 164 104) (end 168 104) (angle 90) (layer Edge.Cuts) (width 0.1))
 (segment (start 148 104) (end 156 96) (width 0.6096) (layer F.Cu) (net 3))
 (segment (start 148 88) (end 156 96) (width 0.6096) (layer F.Cu) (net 3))
 (segment (start 152.25 84.75) (end 151.75 85.25) (width 0.6096) (layer F.Cu) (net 3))
 (segment (start 152.25 83.5) (end 152.25 82.75) (width 0.6096) (layer F.Cu) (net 3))
 (segment (start 152 82) (end 152.25 82.25) (width 0.4064) (layer F.Cu) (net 3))
 (segment (start 152.25 82.25) (end 152.25 82.75) (width 0.4064) (layer F.Cu) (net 3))
 (segment (start 152 75) (end 152 82) (width 0.4064) (layer F.Cu) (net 3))
 (segment (start 152.25 84.75) (end 152.25 83.5) (width 0.3048) (layer F.Cu) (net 3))
 (segment (start 150.75 85.25) (end 148 88) (width 0.6096) (layer F.Cu) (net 3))
 (segment (start 151.75 85.25) (end 150.75 85.25) (width 0.6096) (layer F.Cu) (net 3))
 (segment (start 150.35 75) (end 152 75) (width 0.4064) (layer F.Cu) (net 3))
 (segment (start 152 64.8) (end 152 75) (width 0.6096) (layer B.Cu) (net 3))
 (segment (start 148 64) (end 151.2 64) (width 0.6096) (layer B.Cu) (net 3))
 (segment (start 151.2 64) (end 152 64.8) (width 0.6096) (layer B.Cu) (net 3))
 (segment (start 148 88) (end 149 88) (width 0.4064) (layer F.Cu) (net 3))
 (segment (start 145 96) (end 145 93) (width 0.6096) (layer F.Cu) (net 1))
 (segment (start 165.75 92.5) (end 167 93.75) (width 0.6096) (layer F.Cu) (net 1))
 (via (at 165.75 92.5) (size 0.6) (drill 0.4) (layers F.Cu B.Cu) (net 1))
 (segment (start 145.5 92.5) (end 165.75 92.5) (width 0.6096) (layer B.Cu) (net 1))
 (via (at 145.5 92.5) (size 0.6) (drill 0.4) (layers F.Cu B.Cu) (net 1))
 (segment (start 145 93) (end 145.5 92.5) (width 0.6096) (layer F.Cu) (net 1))
 (segment (start 167 93.75) (end 167 96) (width 0.6096) (layer F.Cu) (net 1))
 (segment (start 145 96) (end 145 99) (width 0.6096) (layer F.Cu) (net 1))
 (segment (start 165.75 99.75) (end 167 98.5) (width 0.6096) (layer F.Cu) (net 1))
 (via (at 165.75 99.75) (size 0.6) (drill 0.4) (layers F.Cu B.Cu) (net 1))
 (segment (start 145.75 99.75) (end 165.75 99.75) (width 0.6096) (layer B.Cu) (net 1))
 (segment (start 145.5 99.5) (end 145.75 99.75) (width 0.6096) (layer B.Cu) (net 1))
 (via (at 145.5 99.5) (size 0.6) (drill 0.4) (layers F.Cu B.Cu) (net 1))
 (segment (start 145 99) (end 145.5 99.5) (width 0.6096) (layer F.Cu) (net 1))
 (segment (start 167 98.5) (end 167 96) (width 0.6096) (layer F.Cu) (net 1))
 (segment (start 167 96) (end 167 101) (width 0.6096) (layer F.Cu) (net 1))
 (segment (start 167 101) (end 164 104) (width 0.6096) (layer F.Cu) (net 1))
 (segment (start 167 96) (end 167 91) (width 0.6096) (layer F.Cu) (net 1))
 (segment (start 167 91) (end 164 88) (width 0.6096) (layer F.Cu) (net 1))
 (segment (start 153.25 85) (end 157.25 85) (width 0.3048) (layer F.Cu) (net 1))
 (segment (start 152.25 86) (end 153.25 85) (width 0.4064) (layer F.Cu) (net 1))
 (via (at 152.25 86) (size 0.6) (drill 0.4) (layers F.Cu B.Cu) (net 1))
 (segment (start 159.25 87) (end 163 87) (width 0.3048) (layer F.Cu) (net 1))
 (segment (start 157.25 85) (end 159.25 87) (width 0.3048) (layer F.Cu) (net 1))
 (segment (start 163 87) (end 164 88) (width 0.3048) (layer F.Cu) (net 1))
 (segment (start 161 77.25) (end 161.25 77.5) (width 0.4064) (layer B.Cu) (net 1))
 (segment (start 160.5 76.75) (end 159.5 76.75) (width 0.3048) (layer B.Cu) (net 1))
 (segment (start 154.75 75.75) (end 157.25 75.75) (width 0.4064) (layer B.Cu) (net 1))
 (segment (start 152.25 82.25) (end 152 82) (width 0.4064) (layer B.Cu) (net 1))
 (segment (start 152.25 82.75) (end 152.25 83.5) (width 0.6096) (layer B.Cu) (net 1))
 (segment (start 152.25 86) (end 152.25 85) (width 0.6096) (layer B.Cu) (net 1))
 (segment (start 152.25 83.5) (end 152.25 85) (width 0.3048) (layer B.Cu) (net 1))
 (segment (start 154.75 75.75) (end 152 78.5) (width 0.4064) (layer B.Cu) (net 1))
 (segment (start 152 78.5) (end 152 82) (width 0.4064) (layer B.Cu) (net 1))
 (segment (start 152.25 82.75) (end 152.25 82.25) (width 0.4064) (layer B.Cu) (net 1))
 (segment (start 158.25 76.75) (end 158.5 76.75) (width 0.4064) (layer B.Cu) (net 1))
 (segment (start 157.25 75.75) (end 158.25 76.75) (width 0.4064) (layer B.Cu) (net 1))
 (segment (start 159.5 76.75) (end 158.5 76.75) (width 0.6096) (layer B.Cu) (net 1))
 (segment (start 161 77.25) (end 160.5 76.75) (width 0.6096) (layer B.Cu) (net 1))
 (segment (start 161.5 77.75) (end 161.75 77.75) (width 0.4064) (layer B.Cu) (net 1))
 (segment (start 161.25 77.5) (end 161.5 77.75) (width 0.4064) (layer B.Cu) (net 1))
 (segment (start 161.75 77.75) (end 164 80) (width 0.4064) (layer B.Cu) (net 1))
 (segment (start 152.25 90) (end 152.25 86) (width 0.4064) (layer B.Cu) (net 1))
 (segment (start 150 92.25) (end 152.25 90) (width 0.4064) (layer B.Cu) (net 1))
 (segment (start 167.43 96) (end 167.43 98.32) (width 0.4064) (layer F.Cu) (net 1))
 (segment (start 167 95.57) (end 167.43 96) (width 0.4064) (layer F.Cu) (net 1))
 (segment (start 164 80) (end 163.75 80) (width 0.4064) (layer B.Cu) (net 1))
 (segment (start 166.54 75.81) (end 166.54 77.46) (width 0.4064) (layer F.Cu) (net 1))
 (segment (start 166.54 77.46) (end 164 80) (width 0.4064) (layer F.Cu) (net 1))
 (segment (start 166.54 68.19) (end 166.54 68.54) (width 0.4064) (layer F.Cu) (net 1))
 (segment (start 166.54 68.54) (end 167 69) (width 0.4064) (layer F.Cu) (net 1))
 (segment (start 167 69) (end 167 75.35) (width 0.4064) (layer F.Cu) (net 1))
 (segment (start 167 75.35) (end 166.54 75.81) (width 0.4064) (layer F.Cu) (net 1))
 (segment (start 160.5 76.75) (end 160.52 76.75) (width 0.6096) (layer F.Cu) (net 2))
 (segment (start 159.5 76.75) (end 158.5 76.75) (width 0.6096) (layer F.Cu) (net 2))
 (segment (start 155 75.75) (end 157.25 75.75) (width 0.4064) (layer F.Cu) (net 2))
 (segment (start 157.25 75.75) (end 158.25 76.75) (width 0.4064) (layer F.Cu) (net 2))
 (segment (start 158.25 76.75) (end 158.5 76.75) (width 0.4064) (layer F.Cu) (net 2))
 (segment (start 154.25 75) (end 155 75.75) (width 0.4064) (layer F.Cu) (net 2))
 (segment (start 160.5 76.75) (end 159.5 76.75) (width 0.3048) (layer F.Cu) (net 2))
 (segment (start 160.52 76.75) (end 161.46 75.81) (width 0.6096) (layer F.Cu) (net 2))
 (segment (start 153.65 75) (end 154.25 75) (width 0.4064) (layer F.Cu) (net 2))
 (segment (start 153.65 75) (end 153.65 77.65) (width 0.4064) (layer F.Cu) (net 2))
 (segment (start 153.65 77.65) (end 156 80) (width 0.4064) (layer F.Cu) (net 2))
 (segment (start 153.9 75.25) (end 153.65 75) (width 0.4064) (layer F.Cu) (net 2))
 (segment (start 161.46 69.54) (end 161 70) (width 0.4064) (layer F.Cu) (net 2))
 (segment (start 161.46 68.19) (end 161.46 69.54) (width 0.4064) (layer F.Cu) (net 2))
 (segment (start 161 70) (end 161 75.35) (width 0.4064) (layer F.Cu) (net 2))
 (segment (start 161 75.35) (end 161.46 75.81) (width 0.4064) (layer F.Cu) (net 2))
 (segment (start 161.46 68.19) (end 161.46 66.54) (width 0.4064) (layer F.Cu) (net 2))
 (segment (start 161.46 66.54) (end 164 64) (width 0.4064) (layer F.Cu) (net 2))
 (segment (start 153.65 75) (end 153.65 74.65) (width 0.4064) (layer F.Cu) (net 2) (status 10)))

